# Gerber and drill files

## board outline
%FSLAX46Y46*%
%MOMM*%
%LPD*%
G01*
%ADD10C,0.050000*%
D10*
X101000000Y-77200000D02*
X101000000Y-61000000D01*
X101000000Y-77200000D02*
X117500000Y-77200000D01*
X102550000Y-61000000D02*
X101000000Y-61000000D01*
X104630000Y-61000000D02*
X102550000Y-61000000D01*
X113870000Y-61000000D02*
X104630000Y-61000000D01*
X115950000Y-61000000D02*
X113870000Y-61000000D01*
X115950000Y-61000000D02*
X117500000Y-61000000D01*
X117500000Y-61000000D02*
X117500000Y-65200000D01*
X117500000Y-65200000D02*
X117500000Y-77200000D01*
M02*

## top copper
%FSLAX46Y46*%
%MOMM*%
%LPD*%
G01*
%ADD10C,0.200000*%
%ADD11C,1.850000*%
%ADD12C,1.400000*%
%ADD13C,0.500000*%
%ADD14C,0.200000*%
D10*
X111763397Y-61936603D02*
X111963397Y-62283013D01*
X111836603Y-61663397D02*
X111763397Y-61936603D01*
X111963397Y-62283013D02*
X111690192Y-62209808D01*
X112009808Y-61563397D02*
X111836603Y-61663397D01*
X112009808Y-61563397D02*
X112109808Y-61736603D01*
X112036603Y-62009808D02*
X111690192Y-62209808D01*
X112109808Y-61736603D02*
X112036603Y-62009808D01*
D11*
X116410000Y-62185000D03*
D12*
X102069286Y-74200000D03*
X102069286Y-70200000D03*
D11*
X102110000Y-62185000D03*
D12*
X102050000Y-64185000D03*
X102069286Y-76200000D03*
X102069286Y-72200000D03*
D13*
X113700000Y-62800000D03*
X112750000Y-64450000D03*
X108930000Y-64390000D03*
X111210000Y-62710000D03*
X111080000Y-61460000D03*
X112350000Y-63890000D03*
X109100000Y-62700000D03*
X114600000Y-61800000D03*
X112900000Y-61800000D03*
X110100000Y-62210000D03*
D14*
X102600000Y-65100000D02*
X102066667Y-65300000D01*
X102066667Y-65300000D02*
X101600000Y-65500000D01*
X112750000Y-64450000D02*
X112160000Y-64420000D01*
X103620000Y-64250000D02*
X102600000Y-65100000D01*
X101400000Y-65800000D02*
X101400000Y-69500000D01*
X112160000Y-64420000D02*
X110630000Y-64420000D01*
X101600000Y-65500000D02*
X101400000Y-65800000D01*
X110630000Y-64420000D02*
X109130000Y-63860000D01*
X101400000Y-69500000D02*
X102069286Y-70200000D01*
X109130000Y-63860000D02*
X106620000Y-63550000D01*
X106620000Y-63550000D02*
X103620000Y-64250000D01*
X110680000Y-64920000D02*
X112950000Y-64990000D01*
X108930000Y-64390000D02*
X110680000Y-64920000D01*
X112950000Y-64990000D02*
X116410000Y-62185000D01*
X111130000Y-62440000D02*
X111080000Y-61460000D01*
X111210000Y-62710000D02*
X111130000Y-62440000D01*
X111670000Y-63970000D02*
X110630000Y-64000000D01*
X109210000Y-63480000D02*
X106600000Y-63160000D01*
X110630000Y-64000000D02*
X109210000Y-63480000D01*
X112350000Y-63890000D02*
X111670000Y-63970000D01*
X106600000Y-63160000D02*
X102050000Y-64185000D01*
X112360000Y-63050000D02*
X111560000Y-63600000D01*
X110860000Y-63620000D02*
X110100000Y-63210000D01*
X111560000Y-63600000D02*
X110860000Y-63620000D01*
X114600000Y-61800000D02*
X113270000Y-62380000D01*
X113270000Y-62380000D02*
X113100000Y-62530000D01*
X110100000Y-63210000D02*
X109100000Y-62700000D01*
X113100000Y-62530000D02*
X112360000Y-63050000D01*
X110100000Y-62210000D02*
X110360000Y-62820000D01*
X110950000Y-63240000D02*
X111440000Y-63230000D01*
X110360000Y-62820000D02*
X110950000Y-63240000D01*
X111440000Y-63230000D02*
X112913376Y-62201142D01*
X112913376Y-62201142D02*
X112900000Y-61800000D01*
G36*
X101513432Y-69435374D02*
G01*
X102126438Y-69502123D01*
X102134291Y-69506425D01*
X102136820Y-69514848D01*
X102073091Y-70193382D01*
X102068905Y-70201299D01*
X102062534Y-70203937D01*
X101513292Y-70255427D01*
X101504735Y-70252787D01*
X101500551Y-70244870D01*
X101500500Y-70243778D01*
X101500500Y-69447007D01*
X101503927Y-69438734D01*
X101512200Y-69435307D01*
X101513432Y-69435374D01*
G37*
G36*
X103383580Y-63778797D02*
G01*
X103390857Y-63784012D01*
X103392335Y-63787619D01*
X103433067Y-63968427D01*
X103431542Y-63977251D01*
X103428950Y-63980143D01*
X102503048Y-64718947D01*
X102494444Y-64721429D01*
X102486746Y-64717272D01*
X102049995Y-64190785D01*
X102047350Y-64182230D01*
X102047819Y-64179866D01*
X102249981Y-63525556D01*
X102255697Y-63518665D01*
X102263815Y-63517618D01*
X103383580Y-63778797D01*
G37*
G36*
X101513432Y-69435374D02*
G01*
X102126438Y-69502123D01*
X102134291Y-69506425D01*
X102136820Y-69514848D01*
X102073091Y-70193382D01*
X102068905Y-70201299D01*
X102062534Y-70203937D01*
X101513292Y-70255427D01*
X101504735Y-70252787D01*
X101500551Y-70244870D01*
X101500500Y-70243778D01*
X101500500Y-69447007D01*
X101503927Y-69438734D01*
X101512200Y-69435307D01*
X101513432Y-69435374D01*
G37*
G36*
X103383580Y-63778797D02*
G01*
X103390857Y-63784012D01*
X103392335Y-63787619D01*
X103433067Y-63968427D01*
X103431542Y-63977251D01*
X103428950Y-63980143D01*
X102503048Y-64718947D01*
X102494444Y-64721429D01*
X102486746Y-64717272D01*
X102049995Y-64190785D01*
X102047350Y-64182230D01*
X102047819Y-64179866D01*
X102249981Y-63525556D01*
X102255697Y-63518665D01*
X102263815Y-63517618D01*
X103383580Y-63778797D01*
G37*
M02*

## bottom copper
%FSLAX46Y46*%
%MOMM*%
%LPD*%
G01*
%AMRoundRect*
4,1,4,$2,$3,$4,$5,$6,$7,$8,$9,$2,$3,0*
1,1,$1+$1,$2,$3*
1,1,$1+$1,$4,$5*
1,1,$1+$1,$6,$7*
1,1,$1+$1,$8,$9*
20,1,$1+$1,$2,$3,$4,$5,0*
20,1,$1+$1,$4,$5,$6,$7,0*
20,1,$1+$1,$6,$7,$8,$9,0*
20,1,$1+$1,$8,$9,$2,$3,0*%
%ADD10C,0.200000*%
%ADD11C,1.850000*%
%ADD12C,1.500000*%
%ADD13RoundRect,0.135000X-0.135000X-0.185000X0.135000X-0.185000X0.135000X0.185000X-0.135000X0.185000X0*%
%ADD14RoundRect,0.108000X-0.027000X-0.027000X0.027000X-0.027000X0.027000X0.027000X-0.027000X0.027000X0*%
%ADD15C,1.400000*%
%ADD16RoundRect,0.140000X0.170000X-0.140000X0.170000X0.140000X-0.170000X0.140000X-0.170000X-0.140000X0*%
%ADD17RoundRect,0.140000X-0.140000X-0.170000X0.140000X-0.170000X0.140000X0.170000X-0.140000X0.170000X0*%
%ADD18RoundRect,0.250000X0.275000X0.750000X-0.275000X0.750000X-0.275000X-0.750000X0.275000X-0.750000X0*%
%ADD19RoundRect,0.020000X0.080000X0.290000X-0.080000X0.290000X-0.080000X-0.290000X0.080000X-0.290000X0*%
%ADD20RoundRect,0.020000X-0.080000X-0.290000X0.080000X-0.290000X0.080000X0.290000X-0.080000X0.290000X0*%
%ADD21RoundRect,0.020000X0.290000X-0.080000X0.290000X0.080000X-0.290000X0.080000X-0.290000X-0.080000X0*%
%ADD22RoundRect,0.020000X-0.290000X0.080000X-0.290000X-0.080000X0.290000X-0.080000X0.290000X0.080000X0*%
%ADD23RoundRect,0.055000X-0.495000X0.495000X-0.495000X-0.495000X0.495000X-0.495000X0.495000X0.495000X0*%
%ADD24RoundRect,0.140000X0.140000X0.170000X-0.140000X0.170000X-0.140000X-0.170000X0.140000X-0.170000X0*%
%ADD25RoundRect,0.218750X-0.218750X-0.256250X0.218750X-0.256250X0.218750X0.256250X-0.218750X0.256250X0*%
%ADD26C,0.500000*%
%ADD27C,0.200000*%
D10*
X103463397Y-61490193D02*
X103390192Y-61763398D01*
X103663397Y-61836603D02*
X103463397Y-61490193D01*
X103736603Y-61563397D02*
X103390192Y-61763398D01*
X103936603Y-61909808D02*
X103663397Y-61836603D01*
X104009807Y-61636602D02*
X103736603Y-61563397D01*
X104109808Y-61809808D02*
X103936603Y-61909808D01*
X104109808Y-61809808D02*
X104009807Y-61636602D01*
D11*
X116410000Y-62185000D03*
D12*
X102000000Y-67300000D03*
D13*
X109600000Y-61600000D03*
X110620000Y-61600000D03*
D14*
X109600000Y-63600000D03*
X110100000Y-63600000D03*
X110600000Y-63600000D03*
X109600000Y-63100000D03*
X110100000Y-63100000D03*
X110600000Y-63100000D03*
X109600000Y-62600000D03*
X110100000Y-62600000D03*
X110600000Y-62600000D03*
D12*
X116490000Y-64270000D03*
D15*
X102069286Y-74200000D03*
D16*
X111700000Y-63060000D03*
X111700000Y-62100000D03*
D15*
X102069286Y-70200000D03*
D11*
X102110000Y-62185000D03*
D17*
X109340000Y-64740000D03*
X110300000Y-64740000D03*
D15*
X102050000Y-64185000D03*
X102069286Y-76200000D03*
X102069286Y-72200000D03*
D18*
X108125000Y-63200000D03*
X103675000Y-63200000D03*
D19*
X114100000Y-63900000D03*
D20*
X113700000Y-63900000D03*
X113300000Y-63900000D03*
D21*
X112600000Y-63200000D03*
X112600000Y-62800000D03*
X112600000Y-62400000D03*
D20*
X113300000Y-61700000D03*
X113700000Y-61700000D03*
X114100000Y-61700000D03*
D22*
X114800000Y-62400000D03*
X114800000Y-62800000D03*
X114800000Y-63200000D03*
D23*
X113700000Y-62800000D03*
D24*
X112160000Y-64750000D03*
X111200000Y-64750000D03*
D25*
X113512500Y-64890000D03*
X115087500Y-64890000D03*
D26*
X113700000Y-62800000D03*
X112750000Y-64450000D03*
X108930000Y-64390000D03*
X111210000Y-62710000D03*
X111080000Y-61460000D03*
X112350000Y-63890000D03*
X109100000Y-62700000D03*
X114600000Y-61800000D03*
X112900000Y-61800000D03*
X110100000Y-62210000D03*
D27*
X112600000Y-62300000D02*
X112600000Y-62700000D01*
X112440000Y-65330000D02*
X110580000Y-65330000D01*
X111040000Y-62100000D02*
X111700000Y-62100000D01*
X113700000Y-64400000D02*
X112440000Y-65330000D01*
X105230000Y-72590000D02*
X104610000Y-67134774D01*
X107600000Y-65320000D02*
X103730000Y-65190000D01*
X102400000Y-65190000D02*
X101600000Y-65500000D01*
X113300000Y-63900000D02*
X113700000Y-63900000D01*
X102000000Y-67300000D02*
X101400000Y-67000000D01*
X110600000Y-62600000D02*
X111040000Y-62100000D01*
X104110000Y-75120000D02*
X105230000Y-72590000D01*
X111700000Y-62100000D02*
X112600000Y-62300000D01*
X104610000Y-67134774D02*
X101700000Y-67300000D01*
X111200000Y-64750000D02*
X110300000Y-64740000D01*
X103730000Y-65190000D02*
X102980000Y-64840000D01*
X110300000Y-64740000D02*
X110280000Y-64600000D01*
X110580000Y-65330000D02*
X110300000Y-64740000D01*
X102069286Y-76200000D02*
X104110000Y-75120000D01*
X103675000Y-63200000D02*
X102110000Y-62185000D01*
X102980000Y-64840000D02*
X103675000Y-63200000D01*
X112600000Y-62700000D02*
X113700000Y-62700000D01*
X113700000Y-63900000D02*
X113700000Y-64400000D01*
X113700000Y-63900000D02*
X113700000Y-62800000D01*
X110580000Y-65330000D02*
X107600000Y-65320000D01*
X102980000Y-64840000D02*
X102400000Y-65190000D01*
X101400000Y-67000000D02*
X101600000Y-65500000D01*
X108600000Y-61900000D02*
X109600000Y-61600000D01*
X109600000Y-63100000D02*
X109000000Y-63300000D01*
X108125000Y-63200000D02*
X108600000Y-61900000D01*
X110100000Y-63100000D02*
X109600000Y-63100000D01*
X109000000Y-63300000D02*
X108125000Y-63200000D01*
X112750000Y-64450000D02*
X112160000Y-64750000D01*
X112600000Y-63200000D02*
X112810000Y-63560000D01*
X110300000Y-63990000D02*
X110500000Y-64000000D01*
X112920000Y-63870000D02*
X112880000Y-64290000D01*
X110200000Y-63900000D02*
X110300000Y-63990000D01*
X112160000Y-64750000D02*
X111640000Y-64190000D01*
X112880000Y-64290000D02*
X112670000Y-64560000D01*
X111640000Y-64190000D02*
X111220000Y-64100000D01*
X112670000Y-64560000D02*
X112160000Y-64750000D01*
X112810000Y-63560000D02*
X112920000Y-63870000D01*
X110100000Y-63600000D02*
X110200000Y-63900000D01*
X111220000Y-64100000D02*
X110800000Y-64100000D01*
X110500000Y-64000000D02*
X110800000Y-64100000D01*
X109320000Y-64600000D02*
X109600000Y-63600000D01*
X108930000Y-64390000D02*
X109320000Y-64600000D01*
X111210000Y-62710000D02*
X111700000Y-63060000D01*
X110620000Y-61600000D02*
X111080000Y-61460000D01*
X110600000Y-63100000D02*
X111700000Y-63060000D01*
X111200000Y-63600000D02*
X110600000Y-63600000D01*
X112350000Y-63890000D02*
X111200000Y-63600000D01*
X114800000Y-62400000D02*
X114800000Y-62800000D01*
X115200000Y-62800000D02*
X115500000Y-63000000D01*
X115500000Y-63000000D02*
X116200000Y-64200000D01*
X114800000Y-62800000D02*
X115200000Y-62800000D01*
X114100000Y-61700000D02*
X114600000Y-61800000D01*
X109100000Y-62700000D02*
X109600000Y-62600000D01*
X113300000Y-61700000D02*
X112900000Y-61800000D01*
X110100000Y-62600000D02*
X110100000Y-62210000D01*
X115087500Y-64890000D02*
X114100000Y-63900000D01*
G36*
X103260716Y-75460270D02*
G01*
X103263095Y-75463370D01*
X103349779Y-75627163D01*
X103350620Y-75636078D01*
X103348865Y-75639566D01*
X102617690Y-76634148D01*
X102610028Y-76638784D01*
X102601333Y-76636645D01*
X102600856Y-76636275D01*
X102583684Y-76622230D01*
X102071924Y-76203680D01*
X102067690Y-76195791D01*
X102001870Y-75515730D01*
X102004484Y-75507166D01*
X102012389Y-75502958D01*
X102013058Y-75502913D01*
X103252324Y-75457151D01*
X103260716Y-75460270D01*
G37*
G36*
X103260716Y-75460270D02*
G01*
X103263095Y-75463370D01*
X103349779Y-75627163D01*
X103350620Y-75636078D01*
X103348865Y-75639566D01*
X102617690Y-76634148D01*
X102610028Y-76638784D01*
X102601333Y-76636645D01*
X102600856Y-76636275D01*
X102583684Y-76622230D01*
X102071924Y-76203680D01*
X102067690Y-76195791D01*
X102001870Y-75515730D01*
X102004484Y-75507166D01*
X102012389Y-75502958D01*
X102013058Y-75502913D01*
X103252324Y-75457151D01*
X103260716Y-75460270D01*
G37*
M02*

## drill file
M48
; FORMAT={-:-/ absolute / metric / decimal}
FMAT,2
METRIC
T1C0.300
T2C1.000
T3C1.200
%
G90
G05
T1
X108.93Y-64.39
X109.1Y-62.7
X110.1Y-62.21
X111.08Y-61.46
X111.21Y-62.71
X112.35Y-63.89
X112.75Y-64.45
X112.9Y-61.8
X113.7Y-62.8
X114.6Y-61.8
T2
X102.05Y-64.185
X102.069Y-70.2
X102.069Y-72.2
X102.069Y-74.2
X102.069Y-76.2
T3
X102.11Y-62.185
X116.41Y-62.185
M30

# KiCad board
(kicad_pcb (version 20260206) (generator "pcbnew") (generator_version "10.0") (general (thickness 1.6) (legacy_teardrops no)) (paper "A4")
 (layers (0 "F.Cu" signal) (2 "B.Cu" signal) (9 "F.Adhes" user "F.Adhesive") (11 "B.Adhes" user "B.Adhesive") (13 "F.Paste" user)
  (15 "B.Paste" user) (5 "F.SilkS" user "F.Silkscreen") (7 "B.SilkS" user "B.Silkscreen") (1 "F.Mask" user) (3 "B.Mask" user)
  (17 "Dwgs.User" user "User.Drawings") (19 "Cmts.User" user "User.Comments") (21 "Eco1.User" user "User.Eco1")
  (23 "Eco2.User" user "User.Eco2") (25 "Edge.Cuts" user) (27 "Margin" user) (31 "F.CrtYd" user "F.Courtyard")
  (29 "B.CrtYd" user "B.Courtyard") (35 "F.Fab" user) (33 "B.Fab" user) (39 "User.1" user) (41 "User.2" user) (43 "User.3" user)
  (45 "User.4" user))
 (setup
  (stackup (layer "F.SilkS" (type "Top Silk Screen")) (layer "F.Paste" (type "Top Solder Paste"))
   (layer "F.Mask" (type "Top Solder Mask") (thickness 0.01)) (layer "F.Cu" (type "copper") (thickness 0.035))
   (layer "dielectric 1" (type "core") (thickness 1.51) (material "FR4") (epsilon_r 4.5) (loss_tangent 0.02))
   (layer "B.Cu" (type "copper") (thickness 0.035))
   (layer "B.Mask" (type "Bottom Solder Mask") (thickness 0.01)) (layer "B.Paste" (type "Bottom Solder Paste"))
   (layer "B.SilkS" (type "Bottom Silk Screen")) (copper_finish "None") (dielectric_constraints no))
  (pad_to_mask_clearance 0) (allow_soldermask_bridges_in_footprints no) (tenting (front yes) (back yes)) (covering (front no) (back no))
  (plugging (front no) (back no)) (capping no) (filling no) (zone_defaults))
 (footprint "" (layer "F.Cu") (at 116.41 62.185)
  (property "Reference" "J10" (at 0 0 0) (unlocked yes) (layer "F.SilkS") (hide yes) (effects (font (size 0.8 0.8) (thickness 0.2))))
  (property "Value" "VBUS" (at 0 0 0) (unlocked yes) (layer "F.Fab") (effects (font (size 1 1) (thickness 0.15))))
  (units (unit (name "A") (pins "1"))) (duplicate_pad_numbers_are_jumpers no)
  (pad "1" thru_hole circle (at 0 0 180) (size 1.85 1.85) (drill 1.2) (layers "*.Cu" "*.Mask") (remove_unused_layers no) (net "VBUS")))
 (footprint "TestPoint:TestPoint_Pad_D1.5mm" (layer "B.Cu") (at 102 67.3 180)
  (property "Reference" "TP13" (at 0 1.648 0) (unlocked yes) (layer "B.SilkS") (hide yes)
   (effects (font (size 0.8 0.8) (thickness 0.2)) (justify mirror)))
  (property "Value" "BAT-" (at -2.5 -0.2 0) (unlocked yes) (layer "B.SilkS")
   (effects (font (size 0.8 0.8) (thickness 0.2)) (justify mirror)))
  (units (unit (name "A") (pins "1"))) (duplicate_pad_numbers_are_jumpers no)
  (pad "1" smd circle (at 0 0 180) (size 1.5 1.5) (layers "B.Cu" "B.Mask") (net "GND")))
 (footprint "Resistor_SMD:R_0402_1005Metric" (layer "B.Cu") (at 110.11 61.6)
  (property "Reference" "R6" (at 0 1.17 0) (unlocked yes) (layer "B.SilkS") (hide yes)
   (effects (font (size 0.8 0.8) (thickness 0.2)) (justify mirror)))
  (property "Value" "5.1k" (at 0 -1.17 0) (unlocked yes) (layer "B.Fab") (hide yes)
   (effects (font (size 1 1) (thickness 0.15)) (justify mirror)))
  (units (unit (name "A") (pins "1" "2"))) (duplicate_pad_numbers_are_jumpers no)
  (pad "1" smd roundrect (at -0.51 0) (size 0.54 0.64) (layers "B.Cu" "B.Mask" "B.Paste") (roundrect_rratio 0.25) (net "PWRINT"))
  (pad "2" smd roundrect (at 0.51 0) (size 0.54 0.64) (layers "B.Cu" "B.Mask" "B.Paste") (roundrect_rratio 0.25) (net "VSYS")))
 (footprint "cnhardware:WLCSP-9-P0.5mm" (layer "B.Cu") (at 110.1 63.1)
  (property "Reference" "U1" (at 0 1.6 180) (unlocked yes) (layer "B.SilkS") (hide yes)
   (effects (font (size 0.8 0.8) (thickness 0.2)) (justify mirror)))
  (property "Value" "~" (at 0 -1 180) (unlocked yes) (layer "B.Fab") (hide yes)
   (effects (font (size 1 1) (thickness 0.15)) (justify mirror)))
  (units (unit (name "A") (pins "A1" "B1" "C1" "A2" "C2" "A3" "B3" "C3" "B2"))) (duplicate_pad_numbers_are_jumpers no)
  (pad "A1" smd roundrect (at -0.5 0.5) (size 0.27 0.27) (layers "B.Cu" "B.Mask" "B.Paste") (roundrect_rratio 0.4) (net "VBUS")
   (solder_mask_margin 0.01) (thermal_bridge_angle 45))
  (pad "A2" smd roundrect (at 0 0.5) (size 0.27 0.27) (layers "B.Cu" "B.Mask" "B.Paste") (roundrect_rratio 0.4) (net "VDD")
   (solder_mask_margin 0.01) (thermal_bridge_angle 45))
  (pad "A3" smd roundrect (at 0.5 0.5) (size 0.27 0.27) (layers "B.Cu" "B.Mask" "B.Paste") (roundrect_rratio 0.4) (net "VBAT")
   (solder_mask_margin 0.01) (thermal_bridge_angle 45))
  (pad "B1" smd roundrect (at -0.5 0) (size 0.27 0.27) (layers "B.Cu" "B.Mask" "B.Paste") (roundrect_rratio 0.4) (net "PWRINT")
   (solder_mask_margin 0.01) (thermal_bridge_angle 45))
  (pad "B2" smd roundrect (at 0 0) (size 0.27 0.27) (layers "B.Cu" "B.Mask" "B.Paste") (roundrect_rratio 0.4) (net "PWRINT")
   (solder_mask_margin 0.01) (thermal_bridge_angle 45))
  (pad "B3" smd roundrect (at 0.5 0) (size 0.27 0.27) (layers "B.Cu" "B.Mask" "B.Paste") (roundrect_rratio 0.4) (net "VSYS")
   (solder_mask_margin 0.01) (thermal_bridge_angle 45))
  (pad "C1" smd roundrect (at -0.5 -0.5) (size 0.27 0.27) (layers "B.Cu" "B.Mask" "B.Paste") (roundrect_rratio 0.4) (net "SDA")
   (solder_mask_margin 0.01) (thermal_bridge_angle 45))
  (pad "C2" smd roundrect (at 0 -0.5) (size 0.27 0.27) (layers "B.Cu" "B.Mask" "B.Paste") (roundrect_rratio 0.4) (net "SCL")
   (solder_mask_margin 0.01) (thermal_bridge_angle 45))
  (pad "C3" smd roundrect (at 0.5 -0.5) (size 0.27 0.27) (layers "B.Cu" "B.Mask" "B.Paste") (roundrect_rratio 0.4) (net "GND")
   (solder_mask_margin 0.01) (thermal_bridge_angle 45)))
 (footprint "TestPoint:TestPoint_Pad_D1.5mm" (layer "B.Cu") (at 116.49 64.27 180)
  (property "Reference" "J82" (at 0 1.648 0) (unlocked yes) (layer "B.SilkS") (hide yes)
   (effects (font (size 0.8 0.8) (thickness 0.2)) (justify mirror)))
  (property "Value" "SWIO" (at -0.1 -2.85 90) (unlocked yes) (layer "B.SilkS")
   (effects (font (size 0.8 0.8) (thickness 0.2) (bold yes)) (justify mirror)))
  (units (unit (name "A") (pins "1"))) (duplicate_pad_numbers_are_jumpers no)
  (pad "1" smd circle (at 0 0 180) (size 1.5 1.5) (layers "B.Cu" "B.Mask") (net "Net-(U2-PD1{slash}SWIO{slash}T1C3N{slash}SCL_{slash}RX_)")))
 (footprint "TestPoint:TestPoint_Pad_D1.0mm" (layer "B.Cu") (at 102.069286 74.2 180)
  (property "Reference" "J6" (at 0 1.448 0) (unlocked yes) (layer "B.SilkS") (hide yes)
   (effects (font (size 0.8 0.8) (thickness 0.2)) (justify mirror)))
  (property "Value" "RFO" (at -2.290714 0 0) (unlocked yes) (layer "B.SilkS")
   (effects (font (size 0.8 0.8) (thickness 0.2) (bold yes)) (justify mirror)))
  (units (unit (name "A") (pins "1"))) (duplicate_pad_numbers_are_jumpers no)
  (pad "1" thru_hole circle (at 0 0 180) (size 1.4 1.4) (drill 1) (layers "*.Cu" "*.Mask") (remove_unused_layers no)
   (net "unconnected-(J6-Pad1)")
   (teardrops (best_length_ratio 0.5) (max_length 1) (best_width_ratio 1) (max_width 2) (curved_edges no) (filter_ratio 0.9) (enabled yes)
    (allow_two_segments yes) (prefer_zone_connections yes))))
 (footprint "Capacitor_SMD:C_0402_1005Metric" (layer "B.Cu") (at 111.7 62.58 90)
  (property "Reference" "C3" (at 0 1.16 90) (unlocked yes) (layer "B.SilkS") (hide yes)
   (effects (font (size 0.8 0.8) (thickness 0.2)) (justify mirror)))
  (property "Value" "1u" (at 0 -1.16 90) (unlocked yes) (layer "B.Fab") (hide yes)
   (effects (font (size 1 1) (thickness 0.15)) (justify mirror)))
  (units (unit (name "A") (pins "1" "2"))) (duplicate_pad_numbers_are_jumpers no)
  (pad "1" smd roundrect (at -0.48 0 90) (size 0.56 0.62) (layers "B.Cu" "B.Mask" "B.Paste") (roundrect_rratio 0.25) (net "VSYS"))
  (pad "2" smd roundrect (at 0.48 0 90) (size 0.56 0.62) (layers "B.Cu" "B.Mask" "B.Paste") (roundrect_rratio 0.25) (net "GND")))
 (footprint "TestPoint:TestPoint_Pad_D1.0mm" (layer "B.Cu") (at 102.069286 70.2 180)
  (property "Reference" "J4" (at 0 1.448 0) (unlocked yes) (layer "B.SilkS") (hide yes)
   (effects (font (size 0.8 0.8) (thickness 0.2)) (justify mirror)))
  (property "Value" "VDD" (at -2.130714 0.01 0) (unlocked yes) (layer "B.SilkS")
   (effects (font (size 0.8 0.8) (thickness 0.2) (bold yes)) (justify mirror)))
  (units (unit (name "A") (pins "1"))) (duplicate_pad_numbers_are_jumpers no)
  (pad "1" thru_hole circle (at 0 0 180) (size 1.4 1.4) (drill 1) (layers "*.Cu" "*.Mask") (remove_unused_layers no) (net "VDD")
   (teardrops (best_length_ratio 0.5) (max_length 1) (best_width_ratio 1) (max_width 2) (curved_edges no) (filter_ratio 0.9) (enabled yes)
    (allow_two_segments yes) (prefer_zone_connections yes))))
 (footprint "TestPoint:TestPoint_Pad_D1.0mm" (layer "B.Cu") (at 102.11 62.185 180)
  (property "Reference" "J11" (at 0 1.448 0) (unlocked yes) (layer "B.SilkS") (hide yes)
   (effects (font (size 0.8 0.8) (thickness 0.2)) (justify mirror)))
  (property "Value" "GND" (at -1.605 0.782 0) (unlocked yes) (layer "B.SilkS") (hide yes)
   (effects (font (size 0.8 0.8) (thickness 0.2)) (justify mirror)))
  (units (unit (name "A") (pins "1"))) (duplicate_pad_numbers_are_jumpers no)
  (pad "1" thru_hole circle (at 0 0 180) (size 1.85 1.85) (drill 1.2) (layers "*.Cu" "*.Mask") (remove_unused_layers no) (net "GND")))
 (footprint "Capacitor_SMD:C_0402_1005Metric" (layer "B.Cu") (at 109.82 64.74)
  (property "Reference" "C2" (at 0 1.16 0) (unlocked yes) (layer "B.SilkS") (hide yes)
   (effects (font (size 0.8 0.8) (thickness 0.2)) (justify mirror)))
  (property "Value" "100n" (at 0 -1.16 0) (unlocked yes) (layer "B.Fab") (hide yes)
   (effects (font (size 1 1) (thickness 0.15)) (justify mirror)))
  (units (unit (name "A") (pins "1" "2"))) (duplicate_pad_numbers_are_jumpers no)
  (pad "1" smd roundrect (at -0.48 0) (size 0.56 0.62) (layers "B.Cu" "B.Mask" "B.Paste") (roundrect_rratio 0.25) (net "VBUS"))
  (pad "2" smd roundrect (at 0.48 0) (size 0.56 0.62) (layers "B.Cu" "B.Mask" "B.Paste") (roundrect_rratio 0.25) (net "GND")))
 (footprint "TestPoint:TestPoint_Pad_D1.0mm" (layer "B.Cu") (at 102.05 64.185 180)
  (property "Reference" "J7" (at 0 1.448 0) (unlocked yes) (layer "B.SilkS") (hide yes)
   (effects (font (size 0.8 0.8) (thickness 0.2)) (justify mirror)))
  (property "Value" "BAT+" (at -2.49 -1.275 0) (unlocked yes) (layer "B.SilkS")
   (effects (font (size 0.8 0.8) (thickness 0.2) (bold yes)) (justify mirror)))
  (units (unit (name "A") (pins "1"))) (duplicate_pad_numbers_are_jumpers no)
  (pad "1" thru_hole circle (at 0 0 180) (size 1.4 1.4) (drill 1) (layers "*.Cu" "*.Mask") (remove_unused_layers no) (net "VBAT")
   (teardrops (best_length_ratio 0.5) (max_length 1) (best_width_ratio 1) (max_width 2) (curved_edges no) (filter_ratio 0.9) (enabled yes)
    (allow_two_segments yes) (prefer_zone_connections yes))))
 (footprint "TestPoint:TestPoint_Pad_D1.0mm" (layer "B.Cu") (at 102.069286 76.2 180)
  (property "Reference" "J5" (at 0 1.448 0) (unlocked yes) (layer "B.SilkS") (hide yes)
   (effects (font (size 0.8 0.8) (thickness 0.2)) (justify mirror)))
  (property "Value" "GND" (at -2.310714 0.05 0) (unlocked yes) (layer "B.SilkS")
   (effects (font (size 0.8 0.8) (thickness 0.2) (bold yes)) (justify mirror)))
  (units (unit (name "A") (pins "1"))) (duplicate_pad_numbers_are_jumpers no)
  (pad "1" thru_hole circle (at 0 0 180) (size 1.4 1.4) (drill 1) (layers "*.Cu" "*.Mask") (remove_unused_layers no) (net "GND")
   (teardrops (best_length_ratio 0.5) (max_length 1) (best_width_ratio 1) (max_width 2) (curved_edges no) (filter_ratio 0.9) (enabled yes)
    (allow_two_segments yes) (prefer_zone_connections yes))))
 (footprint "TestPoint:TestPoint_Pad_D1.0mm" (layer "B.Cu") (at 102.069286 72.2 180)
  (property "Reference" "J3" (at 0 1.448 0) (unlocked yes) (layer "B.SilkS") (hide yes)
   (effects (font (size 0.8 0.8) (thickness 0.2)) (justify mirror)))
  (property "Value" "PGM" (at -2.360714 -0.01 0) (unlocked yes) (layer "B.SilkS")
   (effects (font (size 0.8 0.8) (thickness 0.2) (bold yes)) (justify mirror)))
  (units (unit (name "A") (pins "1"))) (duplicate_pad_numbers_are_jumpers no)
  (pad "1" thru_hole circle (at 0 0 180) (size 1.4 1.4) (drill 1) (layers "*.Cu" "*.Mask") (remove_unused_layers no)
   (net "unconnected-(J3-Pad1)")
   (teardrops (best_length_ratio 0.5) (max_length 1) (best_width_ratio 1) (max_width 2) (curved_edges no) (filter_ratio 0.9) (enabled yes)
    (allow_two_segments yes) (prefer_zone_connections yes))))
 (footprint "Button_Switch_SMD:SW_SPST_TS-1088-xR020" (layer "B.Cu") (at 105.9 63.2 180)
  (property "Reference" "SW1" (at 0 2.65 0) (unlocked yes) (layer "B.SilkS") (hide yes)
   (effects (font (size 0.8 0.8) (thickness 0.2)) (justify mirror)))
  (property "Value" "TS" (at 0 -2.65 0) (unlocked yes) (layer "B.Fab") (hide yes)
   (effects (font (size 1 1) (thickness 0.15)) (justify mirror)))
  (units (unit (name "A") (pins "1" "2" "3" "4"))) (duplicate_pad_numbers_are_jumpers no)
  (pad "1" smd roundrect (at -2.225 0 180) (size 1.05 2) (layers "B.Cu" "B.Mask" "B.Paste") (roundrect_rratio 0.2380952381) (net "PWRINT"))
  (pad "3" smd roundrect (at 2.225 0 180) (size 1.05 2) (layers "B.Cu" "B.Mask" "B.Paste") (roundrect_rratio 0.2380952381) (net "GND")))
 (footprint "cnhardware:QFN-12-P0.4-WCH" (layer "B.Cu") (at 113.7 62.8 180)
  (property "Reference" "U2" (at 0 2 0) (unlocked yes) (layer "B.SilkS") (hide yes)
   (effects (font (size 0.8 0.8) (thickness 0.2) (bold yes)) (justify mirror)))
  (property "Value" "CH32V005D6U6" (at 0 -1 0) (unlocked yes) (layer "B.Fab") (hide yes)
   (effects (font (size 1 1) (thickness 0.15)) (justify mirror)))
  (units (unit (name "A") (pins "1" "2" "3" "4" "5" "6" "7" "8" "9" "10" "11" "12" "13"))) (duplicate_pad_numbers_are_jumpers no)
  (pad "1" smd roundrect (at -0.4 -1.1 180) (size 0.2 0.62) (layers "B.Cu" "B.Mask" "B.Paste") (roundrect_rratio 0.1) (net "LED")
   (thermal_bridge_angle 45))
  (pad "2" smd roundrect (at 0 -1.1) (size 0.2 0.62) (layers "B.Cu" "B.Mask" "B.Paste") (roundrect_rratio 0.1) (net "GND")
   (thermal_bridge_angle 45))
  (pad "3" smd roundrect (at 0.4 -1.1) (size 0.2 0.62) (layers "B.Cu" "B.Mask" "B.Paste") (roundrect_rratio 0.1) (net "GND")
   (thermal_bridge_angle 45))
  (pad "4" smd roundrect (at 1.1 -0.4 90) (size 0.2 0.62) (layers "B.Cu" "B.Mask" "B.Paste") (roundrect_rratio 0.1) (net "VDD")
   (thermal_bridge_angle 45))
  (pad "5" smd roundrect (at 1.1 0 90) (size 0.2 0.62) (layers "B.Cu" "B.Mask" "B.Paste") (roundrect_rratio 0.1) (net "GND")
   (thermal_bridge_angle 45))
  (pad "6" smd roundrect (at 1.1 0.4 90) (size 0.2 0.62) (layers "B.Cu" "B.Mask" "B.Paste") (roundrect_rratio 0.1) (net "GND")
   (thermal_bridge_angle 45))
  (pad "7" smd roundrect (at 0.4 1.1) (size 0.2 0.62) (layers "B.Cu" "B.Mask" "B.Paste") (roundrect_rratio 0.1) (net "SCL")
   (thermal_bridge_angle 45))
  (pad "8" smd roundrect (at 0 1.1) (size 0.2 0.62) (layers "B.Cu" "B.Mask" "B.Paste") (roundrect_rratio 0.1)
   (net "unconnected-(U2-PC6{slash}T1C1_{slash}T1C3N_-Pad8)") (thermal_bridge_angle 45))
  (pad "9" smd roundrect (at -0.4 1.1) (size 0.2 0.62) (layers "B.Cu" "B.Mask" "B.Paste") (roundrect_rratio 0.1) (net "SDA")
   (thermal_bridge_angle 45))
  (pad "10" smd roundrect (at -1.1 0.4 270) (size 0.2 0.62) (layers "B.Cu" "B.Mask" "B.Paste") (roundrect_rratio 0.1)
   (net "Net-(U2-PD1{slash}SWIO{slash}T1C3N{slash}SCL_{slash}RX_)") (thermal_bridge_angle 45))
  (pad "11" smd roundrect (at -1.1 0 270) (size 0.2 0.62) (layers "B.Cu" "B.Mask" "B.Paste") (roundrect_rratio 0.1)
   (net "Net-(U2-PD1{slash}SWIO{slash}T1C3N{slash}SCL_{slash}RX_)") (thermal_bridge_angle 45))
  (pad "12" smd roundrect (at -1.1 -0.4 270) (size 0.2 0.62) (layers "B.Cu" "B.Mask" "B.Paste") (roundrect_rratio 0.1)
   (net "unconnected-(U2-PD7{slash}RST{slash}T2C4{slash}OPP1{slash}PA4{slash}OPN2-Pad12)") (thermal_bridge_angle 45))
  (pad "13" smd roundrect (at 0 0 270) (size 1.1 1.1) (layers "B.Cu" "B.Mask" "B.Paste") (roundrect_rratio 0.05) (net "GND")
   (thermal_bridge_angle 45)))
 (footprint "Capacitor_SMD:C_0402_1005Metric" (layer "B.Cu") (at 111.68 64.75 180)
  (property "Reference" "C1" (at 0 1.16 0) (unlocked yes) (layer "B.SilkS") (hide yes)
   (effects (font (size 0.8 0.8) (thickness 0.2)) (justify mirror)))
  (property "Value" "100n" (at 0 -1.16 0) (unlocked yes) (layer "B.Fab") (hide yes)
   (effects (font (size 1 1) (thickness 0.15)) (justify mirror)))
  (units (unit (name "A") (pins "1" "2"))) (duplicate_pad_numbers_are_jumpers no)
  (pad "1" smd roundrect (at -0.48 0 180) (size 0.56 0.62) (layers "B.Cu" "B.Mask" "B.Paste") (roundrect_rratio 0.25) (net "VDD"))
  (pad "2" smd roundrect (at 0.48 0 180) (size 0.56 0.62) (layers "B.Cu" "B.Mask" "B.Paste") (roundrect_rratio 0.25) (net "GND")))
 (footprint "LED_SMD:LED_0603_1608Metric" (layer "B.Cu") (at 114.3 64.89)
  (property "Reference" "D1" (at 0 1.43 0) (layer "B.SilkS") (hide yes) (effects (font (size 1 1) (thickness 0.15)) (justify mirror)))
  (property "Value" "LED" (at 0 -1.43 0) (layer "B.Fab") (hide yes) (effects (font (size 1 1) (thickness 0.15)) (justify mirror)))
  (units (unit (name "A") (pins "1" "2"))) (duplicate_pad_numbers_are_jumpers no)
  (pad "1" smd roundrect (at -0.7875 0) (size 0.875 0.95) (layers "B.Cu" "B.Mask" "B.Paste") (roundrect_rratio 0.25) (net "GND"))
  (pad "2" smd roundrect (at 0.7875 0) (size 0.875 0.95) (layers "B.Cu" "B.Mask" "B.Paste") (roundrect_rratio 0.25) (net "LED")))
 (gr_line (start 111.763397 61.936603) (end 111.963397 62.283013) (stroke (width 0.2) (type default)) (layer "F.Cu"))
 (gr_line (start 111.836603 61.663397) (end 111.763397 61.936603) (stroke (width 0.2) (type default)) (layer "F.Cu"))
 (gr_line (start 111.963397 62.283013) (end 111.690192 62.209808) (stroke (width 0.2) (type default)) (layer "F.Cu"))
 (gr_line (start 112.009808 61.563397) (end 111.836603 61.663397) (stroke (width 0.2) (type default)) (layer "F.Cu"))
 (gr_line (start 112.009808 61.563397) (end 112.109808 61.736603) (stroke (width 0.2) (type default)) (layer "F.Cu"))
 (gr_line (start 112.036603 62.009808) (end 111.690192 62.209808) (stroke (width 0.2) (type default)) (layer "F.Cu"))
 (gr_line (start 112.109808 61.736603) (end 112.036603 62.009808) (stroke (width 0.2) (type default)) (layer "F.Cu"))
 (gr_line (start 103.463397 61.490193) (end 103.390192 61.763398) (stroke (width 0.2) (type default)) (layer "B.Cu"))
 (gr_line (start 103.663397 61.836603) (end 103.463397 61.490193) (stroke (width 0.2) (type default)) (layer "B.Cu"))
 (gr_line (start 103.736603 61.563397) (end 103.390192 61.763398) (stroke (width 0.2) (type default)) (layer "B.Cu"))
 (gr_line (start 103.936603 61.909808) (end 103.663397 61.836603) (stroke (width 0.2) (type default)) (layer "B.Cu"))
 (gr_line (start 104.009807 61.636602) (end 103.736603 61.563397) (stroke (width 0.2) (type default)) (layer "B.Cu"))
 (gr_line (start 104.109808 61.809808) (end 103.936603 61.909808) (stroke (width 0.2) (type default)) (layer "B.Cu"))
 (gr_line (start 104.109808 61.809808) (end 104.009807 61.636602) (stroke (width 0.2) (type default)) (layer "B.Cu"))
 (gr_line (start 101 77.2) (end 101 61) (stroke (width 0.05) (type default)) (layer "Edge.Cuts"))
 (gr_line (start 101 77.2) (end 117.5 77.2) (stroke (width 0.05) (type default)) (layer "Edge.Cuts"))
 (gr_line (start 102.55 61) (end 101 61) (stroke (width 0.05) (type default)) (layer "Edge.Cuts"))
 (gr_line (start 104.63 61) (end 102.55 61) (stroke (width 0.05) (type solid)) (layer "Edge.Cuts"))
 (gr_line (start 113.87 61) (end 104.63 61) (stroke (width 0.05) (type default)) (layer "Edge.Cuts"))
 (gr_line (start 115.95 61) (end 113.87 61) (stroke (width 0.05) (type solid)) (layer "Edge.Cuts"))
 (gr_line (start 115.95 61) (end 117.5 61) (stroke (width 0.05) (type default)) (layer "Edge.Cuts"))
 (gr_line (start 117.5 61) (end 117.5 65.2) (stroke (width 0.05) (type solid)) (layer "Edge.Cuts"))
 (gr_line (start 117.5 65.2) (end 117.5 77.2) (stroke (width 0.05) (type default)) (layer "Edge.Cuts"))
 (via (at 113.7 62.8) (size 0.5) (drill 0.3) (layers "F.Cu" "B.Cu") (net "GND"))
 (segment (start 112.6 62.3) (end 112.6 62.7) (width 0.2) (layer "B.Cu") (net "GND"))
 (segment (start 112.44 65.33) (end 110.58 65.33) (width 0.2) (layer "B.Cu") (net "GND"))
 (segment (start 111.04 62.1) (end 111.7 62.1) (width 0.2) (layer "B.Cu") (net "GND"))
 (segment (start 113.7 64.4) (end 112.44 65.33) (width 0.2) (layer "B.Cu") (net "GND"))
 (segment (start 105.23 72.59) (end 104.61 67.134774) (width 0.2) (layer "B.Cu") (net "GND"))
 (segment (start 107.6 65.32) (end 103.73 65.19) (width 0.2) (layer "B.Cu") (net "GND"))
 (segment (start 102.4 65.19) (end 101.6 65.5) (width 0.2) (layer "B.Cu") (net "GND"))
 (segment (start 113.3 63.9) (end 113.7 63.9) (width 0.2) (layer "B.Cu") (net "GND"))
 (segment (start 102 67.3) (end 101.4 67) (width 0.2) (layer "B.Cu") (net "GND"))
 (segment (start 110.6 62.6) (end 111.04 62.1) (width 0.2) (layer "B.Cu") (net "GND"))
 (segment (start 104.11 75.12) (end 105.23 72.59) (width 0.2) (layer "B.Cu") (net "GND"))
 (segment (start 111.7 62.1) (end 112.6 62.3) (width 0.2) (layer "B.Cu") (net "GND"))
 (segment (start 104.61 67.134774) (end 101.7 67.3) (width 0.2) (layer "B.Cu") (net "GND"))
 (segment (start 111.2 64.75) (end 110.3 64.74) (width 0.2) (layer "B.Cu") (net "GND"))
 (segment (start 103.73 65.19) (end 102.98 64.84) (width 0.2) (layer "B.Cu") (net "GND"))
 (segment (start 110.3 64.74) (end 110.28 64.6) (width 0.2) (layer "B.Cu") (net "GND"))
 (segment (start 110.58 65.33) (end 110.3 64.74) (width 0.2) (layer "B.Cu") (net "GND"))
 (segment (start 102.069286 76.2) (end 104.11 75.12) (width 0.2) (layer "B.Cu") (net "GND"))
 (segment (start 103.675 63.2) (end 102.11 62.185) (width 0.2) (layer "B.Cu") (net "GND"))
 (segment (start 102.98 64.84) (end 103.675 63.2) (width 0.2) (layer "B.Cu") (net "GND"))
 (segment (start 112.6 62.7) (end 113.7 62.7) (width 0.2) (layer "B.Cu") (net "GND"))
 (segment (start 113.7 63.9) (end 113.7 64.4) (width 0.2) (layer "B.Cu") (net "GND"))
 (segment (start 113.7 63.9) (end 113.7 62.8) (width 0.2) (layer "B.Cu") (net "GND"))
 (segment (start 110.58 65.33) (end 107.6 65.32) (width 0.2) (layer "B.Cu") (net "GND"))
 (segment (start 102.98 64.84) (end 102.4 65.19) (width 0.2) (layer "B.Cu") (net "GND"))
 (segment (start 101.4 67) (end 101.6 65.5) (width 0.2) (layer "B.Cu") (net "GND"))
 (segment (start 108.6 61.9) (end 109.6 61.6) (width 0.2) (layer "B.Cu") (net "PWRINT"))
 (segment (start 109.6 63.1) (end 109 63.3) (width 0.2) (layer "B.Cu") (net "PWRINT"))
 (segment (start 108.125 63.2) (end 108.6 61.9) (width 0.2) (layer "B.Cu") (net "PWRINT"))
 (segment (start 110.1 63.1) (end 109.6 63.1) (width 0.2) (layer "B.Cu") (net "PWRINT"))
 (segment (start 109 63.3) (end 108.125 63.2) (width 0.2) (layer "B.Cu") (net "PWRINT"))
 (segment (start 102.6 65.1) (end 102.066667 65.3) (width 0.2) (layer "F.Cu") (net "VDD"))
 (segment (start 102.066667 65.3) (end 101.6 65.5) (width 0.2) (layer "F.Cu") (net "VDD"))
 (segment (start 112.75 64.45) (end 112.16 64.42) (width 0.2) (layer "F.Cu") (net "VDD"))
 (segment (start 103.62 64.25) (end 102.6 65.1) (width 0.2) (layer "F.Cu") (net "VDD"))
 (segment (start 101.4 65.8) (end 101.4 69.5) (width 0.2) (layer "F.Cu") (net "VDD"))
 (segment (start 112.16 64.42) (end 110.63 64.42) (width 0.2) (layer "F.Cu") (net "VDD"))
 (segment (start 101.6 65.5) (end 101.4 65.8) (width 0.2) (layer "F.Cu") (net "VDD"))
 (segment (start 110.63 64.42) (end 109.13 63.86) (width 0.2) (layer "F.Cu") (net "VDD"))
 (segment (start 101.4 69.5) (end 102.069286 70.2) (width 0.2) (layer "F.Cu") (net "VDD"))
 (segment (start 109.13 63.86) (end 106.62 63.55) (width 0.2) (layer "F.Cu") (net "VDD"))
 (segment (start 106.62 63.55) (end 103.62 64.25) (width 0.2) (layer "F.Cu") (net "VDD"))
 (via (at 112.75 64.45) (size 0.5) (drill 0.3) (layers "F.Cu" "B.Cu") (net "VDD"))
 (segment (start 112.75 64.45) (end 112.16 64.75) (width 0.2) (layer "B.Cu") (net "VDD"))
 (segment (start 112.6 63.2) (end 112.81 63.56) (width 0.2) (layer "B.Cu") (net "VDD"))
 (segment (start 110.3 63.99) (end 110.5 64) (width 0.2) (layer "B.Cu") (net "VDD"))
 (segment (start 112.92 63.87) (end 112.88 64.29) (width 0.2) (layer "B.Cu") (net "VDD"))
 (segment (start 110.2 63.9) (end 110.3 63.99) (width 0.2) (layer "B.Cu") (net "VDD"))
 (segment (start 112.16 64.75) (end 111.64 64.19) (width 0.2) (layer "B.Cu") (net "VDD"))
 (segment (start 112.88 64.29) (end 112.67 64.56) (width 0.2) (layer "B.Cu") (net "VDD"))
 (segment (start 111.64 64.19) (end 111.22 64.1) (width 0.2) (layer "B.Cu") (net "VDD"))
 (segment (start 112.67 64.56) (end 112.16 64.75) (width 0.2) (layer "B.Cu") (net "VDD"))
 (segment (start 112.81 63.56) (end 112.92 63.87) (width 0.2) (layer "B.Cu") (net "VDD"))
 (segment (start 110.1 63.6) (end 110.2 63.9) (width 0.2) (layer "B.Cu") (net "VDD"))
 (segment (start 111.22 64.1) (end 110.8 64.1) (width 0.2) (layer "B.Cu") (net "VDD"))
 (segment (start 110.5 64) (end 110.8 64.1) (width 0.2) (layer "B.Cu") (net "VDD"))
 (segment (start 110.68 64.92) (end 112.95 64.99) (width 0.2) (layer "F.Cu") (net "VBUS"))
 (segment (start 108.93 64.39) (end 110.68 64.92) (width 0.2) (layer "F.Cu") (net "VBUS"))
 (segment (start 112.95 64.99) (end 116.41 62.185) (width 0.2) (layer "F.Cu") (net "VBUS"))
 (via (at 108.93 64.39) (size 0.5) (drill 0.3) (layers "F.Cu" "B.Cu") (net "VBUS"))
 (segment (start 109.32 64.6) (end 109.6 63.6) (width 0.2) (layer "B.Cu") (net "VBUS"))
 (segment (start 108.93 64.39) (end 109.32 64.6) (width 0.2) (layer "B.Cu") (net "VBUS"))
 (segment (start 111.13 62.44) (end 111.08 61.46) (width 0.2) (layer "F.Cu") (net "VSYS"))
 (segment (start 111.21 62.71) (end 111.13 62.44) (width 0.2) (layer "F.Cu") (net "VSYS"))
 (via (at 111.21 62.71) (size 0.5) (drill 0.3) (layers "F.Cu" "B.Cu") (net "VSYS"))
 (via (at 111.08 61.46) (size 0.5) (drill 0.3) (layers "F.Cu" "B.Cu") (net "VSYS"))
 (segment (start 111.21 62.71) (end 111.7 63.06) (width 0.2) (layer "B.Cu") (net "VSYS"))
 (segment (start 110.62 61.6) (end 111.08 61.46) (width 0.2) (layer "B.Cu") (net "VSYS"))
 (segment (start 110.6 63.1) (end 111.7 63.06) (width 0.2) (layer "B.Cu") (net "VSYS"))
 (segment (start 111.67 63.97) (end 110.63 64) (width 0.2) (layer "F.Cu") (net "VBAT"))
 (segment (start 109.21 63.48) (end 106.6 63.16) (width 0.2) (layer "F.Cu") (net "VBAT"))
 (segment (start 110.63 64) (end 109.21 63.48) (width 0.2) (layer "F.Cu") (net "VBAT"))
 (segment (start 112.35 63.89) (end 111.67 63.97) (width 0.2) (layer "F.Cu") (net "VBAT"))
 (segment (start 106.6 63.16) (end 102.05 64.185) (width 0.2) (layer "F.Cu") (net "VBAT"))
 (via (at 112.35 63.89) (size 0.5) (drill 0.3) (layers "F.Cu" "B.Cu") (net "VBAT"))
 (segment (start 111.2 63.6) (end 110.6 63.6) (width 0.2) (layer "B.Cu") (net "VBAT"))
 (segment (start 112.35 63.89) (end 111.2 63.6) (width 0.2) (layer "B.Cu") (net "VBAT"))
 (segment (start 114.8 62.4) (end 114.8 62.8) (width 0.2) (layer "B.Cu") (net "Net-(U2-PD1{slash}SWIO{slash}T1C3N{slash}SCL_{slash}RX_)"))
 (segment (start 115.2 62.8) (end 115.5 63) (width 0.2) (layer "B.Cu") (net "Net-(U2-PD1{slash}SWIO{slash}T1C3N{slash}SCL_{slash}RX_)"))
 (segment (start 115.5 63) (end 116.2 64.2) (width 0.2) (layer "B.Cu") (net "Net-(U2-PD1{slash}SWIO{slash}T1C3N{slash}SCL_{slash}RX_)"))
 (segment (start 114.8 62.8) (end 115.2 62.8) (width 0.2) (layer "B.Cu") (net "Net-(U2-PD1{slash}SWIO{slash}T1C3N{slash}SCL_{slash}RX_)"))
 (segment (start 112.36 63.05) (end 111.56 63.6) (width 0.2) (layer "F.Cu") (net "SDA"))
 (segment (start 110.86 63.62) (end 110.1 63.21) (width 0.2) (layer "F.Cu") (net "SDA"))
 (segment (start 111.56 63.6) (end 110.86 63.62) (width 0.2) (layer "F.Cu") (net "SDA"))
 (segment (start 114.6 61.8) (end 113.27 62.38) (width 0.2) (layer "F.Cu") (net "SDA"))
 (segment (start 113.27 62.38) (end 113.1 62.53) (width 0.2) (layer "F.Cu") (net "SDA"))
 (segment (start 110.1 63.21) (end 109.1 62.7) (width 0.2) (layer "F.Cu") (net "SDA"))
 (segment (start 113.1 62.53) (end 112.36 63.05) (width 0.2) (layer "F.Cu") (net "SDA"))
 (via (at 109.1 62.7) (size 0.5) (drill 0.3) (layers "F.Cu" "B.Cu") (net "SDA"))
 (via (at 114.6 61.8) (size 0.5) (drill 0.3) (layers "F.Cu" "B.Cu") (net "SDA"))
 (segment (start 114.1 61.7) (end 114.6 61.8) (width 0.2) (layer "B.Cu") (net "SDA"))
 (segment (start 109.1 62.7) (end 109.6 62.6) (width 0.2) (layer "B.Cu") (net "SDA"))
 (segment (start 110.1 62.21) (end 110.36 62.82) (width 0.2) (layer "F.Cu") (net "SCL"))
 (segment (start 110.95 63.24) (end 111.44 63.23) (width 0.2) (layer "F.Cu") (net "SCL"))
 (segment (start 110.36 62.82) (end 110.95 63.24) (width 0.2) (layer "F.Cu") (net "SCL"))
 (segment (start 111.44 63.23) (end 112.913376 62.201142) (width 0.2) (layer "F.Cu") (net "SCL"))
 (segment (start 112.913376 62.201142) (end 112.9 61.8) (width 0.2) (layer "F.Cu") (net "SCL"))
 (via (at 112.9 61.8) (size 0.5) (drill 0.3) (layers "F.Cu" "B.Cu") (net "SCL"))
 (via (at 110.1 62.21) (size 0.5) (drill 0.3) (layers "F.Cu" "B.Cu") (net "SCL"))
 (segment (start 113.3 61.7) (end 112.9 61.8) (width 0.2) (layer "B.Cu") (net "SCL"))
 (segment (start 110.1 62.6) (end 110.1 62.21) (width 0.2) (layer "B.Cu") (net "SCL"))
 (segment (start 115.0875 64.89) (end 114.1 63.9) (width 0.2) (layer "B.Cu") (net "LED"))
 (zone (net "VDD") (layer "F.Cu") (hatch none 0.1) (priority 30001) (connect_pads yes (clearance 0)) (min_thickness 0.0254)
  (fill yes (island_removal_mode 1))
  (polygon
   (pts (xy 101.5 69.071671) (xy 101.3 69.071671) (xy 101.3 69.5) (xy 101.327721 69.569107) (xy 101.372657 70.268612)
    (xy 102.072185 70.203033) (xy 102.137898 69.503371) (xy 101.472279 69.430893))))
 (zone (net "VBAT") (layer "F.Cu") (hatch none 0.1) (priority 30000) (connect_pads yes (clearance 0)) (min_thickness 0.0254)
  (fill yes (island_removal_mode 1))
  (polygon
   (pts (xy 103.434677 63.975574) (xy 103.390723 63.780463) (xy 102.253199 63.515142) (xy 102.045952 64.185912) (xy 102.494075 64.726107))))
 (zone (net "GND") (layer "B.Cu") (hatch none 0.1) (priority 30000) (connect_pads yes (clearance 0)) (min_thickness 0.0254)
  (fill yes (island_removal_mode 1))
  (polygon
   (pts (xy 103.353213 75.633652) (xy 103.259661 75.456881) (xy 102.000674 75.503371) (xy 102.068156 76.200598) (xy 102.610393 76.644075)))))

